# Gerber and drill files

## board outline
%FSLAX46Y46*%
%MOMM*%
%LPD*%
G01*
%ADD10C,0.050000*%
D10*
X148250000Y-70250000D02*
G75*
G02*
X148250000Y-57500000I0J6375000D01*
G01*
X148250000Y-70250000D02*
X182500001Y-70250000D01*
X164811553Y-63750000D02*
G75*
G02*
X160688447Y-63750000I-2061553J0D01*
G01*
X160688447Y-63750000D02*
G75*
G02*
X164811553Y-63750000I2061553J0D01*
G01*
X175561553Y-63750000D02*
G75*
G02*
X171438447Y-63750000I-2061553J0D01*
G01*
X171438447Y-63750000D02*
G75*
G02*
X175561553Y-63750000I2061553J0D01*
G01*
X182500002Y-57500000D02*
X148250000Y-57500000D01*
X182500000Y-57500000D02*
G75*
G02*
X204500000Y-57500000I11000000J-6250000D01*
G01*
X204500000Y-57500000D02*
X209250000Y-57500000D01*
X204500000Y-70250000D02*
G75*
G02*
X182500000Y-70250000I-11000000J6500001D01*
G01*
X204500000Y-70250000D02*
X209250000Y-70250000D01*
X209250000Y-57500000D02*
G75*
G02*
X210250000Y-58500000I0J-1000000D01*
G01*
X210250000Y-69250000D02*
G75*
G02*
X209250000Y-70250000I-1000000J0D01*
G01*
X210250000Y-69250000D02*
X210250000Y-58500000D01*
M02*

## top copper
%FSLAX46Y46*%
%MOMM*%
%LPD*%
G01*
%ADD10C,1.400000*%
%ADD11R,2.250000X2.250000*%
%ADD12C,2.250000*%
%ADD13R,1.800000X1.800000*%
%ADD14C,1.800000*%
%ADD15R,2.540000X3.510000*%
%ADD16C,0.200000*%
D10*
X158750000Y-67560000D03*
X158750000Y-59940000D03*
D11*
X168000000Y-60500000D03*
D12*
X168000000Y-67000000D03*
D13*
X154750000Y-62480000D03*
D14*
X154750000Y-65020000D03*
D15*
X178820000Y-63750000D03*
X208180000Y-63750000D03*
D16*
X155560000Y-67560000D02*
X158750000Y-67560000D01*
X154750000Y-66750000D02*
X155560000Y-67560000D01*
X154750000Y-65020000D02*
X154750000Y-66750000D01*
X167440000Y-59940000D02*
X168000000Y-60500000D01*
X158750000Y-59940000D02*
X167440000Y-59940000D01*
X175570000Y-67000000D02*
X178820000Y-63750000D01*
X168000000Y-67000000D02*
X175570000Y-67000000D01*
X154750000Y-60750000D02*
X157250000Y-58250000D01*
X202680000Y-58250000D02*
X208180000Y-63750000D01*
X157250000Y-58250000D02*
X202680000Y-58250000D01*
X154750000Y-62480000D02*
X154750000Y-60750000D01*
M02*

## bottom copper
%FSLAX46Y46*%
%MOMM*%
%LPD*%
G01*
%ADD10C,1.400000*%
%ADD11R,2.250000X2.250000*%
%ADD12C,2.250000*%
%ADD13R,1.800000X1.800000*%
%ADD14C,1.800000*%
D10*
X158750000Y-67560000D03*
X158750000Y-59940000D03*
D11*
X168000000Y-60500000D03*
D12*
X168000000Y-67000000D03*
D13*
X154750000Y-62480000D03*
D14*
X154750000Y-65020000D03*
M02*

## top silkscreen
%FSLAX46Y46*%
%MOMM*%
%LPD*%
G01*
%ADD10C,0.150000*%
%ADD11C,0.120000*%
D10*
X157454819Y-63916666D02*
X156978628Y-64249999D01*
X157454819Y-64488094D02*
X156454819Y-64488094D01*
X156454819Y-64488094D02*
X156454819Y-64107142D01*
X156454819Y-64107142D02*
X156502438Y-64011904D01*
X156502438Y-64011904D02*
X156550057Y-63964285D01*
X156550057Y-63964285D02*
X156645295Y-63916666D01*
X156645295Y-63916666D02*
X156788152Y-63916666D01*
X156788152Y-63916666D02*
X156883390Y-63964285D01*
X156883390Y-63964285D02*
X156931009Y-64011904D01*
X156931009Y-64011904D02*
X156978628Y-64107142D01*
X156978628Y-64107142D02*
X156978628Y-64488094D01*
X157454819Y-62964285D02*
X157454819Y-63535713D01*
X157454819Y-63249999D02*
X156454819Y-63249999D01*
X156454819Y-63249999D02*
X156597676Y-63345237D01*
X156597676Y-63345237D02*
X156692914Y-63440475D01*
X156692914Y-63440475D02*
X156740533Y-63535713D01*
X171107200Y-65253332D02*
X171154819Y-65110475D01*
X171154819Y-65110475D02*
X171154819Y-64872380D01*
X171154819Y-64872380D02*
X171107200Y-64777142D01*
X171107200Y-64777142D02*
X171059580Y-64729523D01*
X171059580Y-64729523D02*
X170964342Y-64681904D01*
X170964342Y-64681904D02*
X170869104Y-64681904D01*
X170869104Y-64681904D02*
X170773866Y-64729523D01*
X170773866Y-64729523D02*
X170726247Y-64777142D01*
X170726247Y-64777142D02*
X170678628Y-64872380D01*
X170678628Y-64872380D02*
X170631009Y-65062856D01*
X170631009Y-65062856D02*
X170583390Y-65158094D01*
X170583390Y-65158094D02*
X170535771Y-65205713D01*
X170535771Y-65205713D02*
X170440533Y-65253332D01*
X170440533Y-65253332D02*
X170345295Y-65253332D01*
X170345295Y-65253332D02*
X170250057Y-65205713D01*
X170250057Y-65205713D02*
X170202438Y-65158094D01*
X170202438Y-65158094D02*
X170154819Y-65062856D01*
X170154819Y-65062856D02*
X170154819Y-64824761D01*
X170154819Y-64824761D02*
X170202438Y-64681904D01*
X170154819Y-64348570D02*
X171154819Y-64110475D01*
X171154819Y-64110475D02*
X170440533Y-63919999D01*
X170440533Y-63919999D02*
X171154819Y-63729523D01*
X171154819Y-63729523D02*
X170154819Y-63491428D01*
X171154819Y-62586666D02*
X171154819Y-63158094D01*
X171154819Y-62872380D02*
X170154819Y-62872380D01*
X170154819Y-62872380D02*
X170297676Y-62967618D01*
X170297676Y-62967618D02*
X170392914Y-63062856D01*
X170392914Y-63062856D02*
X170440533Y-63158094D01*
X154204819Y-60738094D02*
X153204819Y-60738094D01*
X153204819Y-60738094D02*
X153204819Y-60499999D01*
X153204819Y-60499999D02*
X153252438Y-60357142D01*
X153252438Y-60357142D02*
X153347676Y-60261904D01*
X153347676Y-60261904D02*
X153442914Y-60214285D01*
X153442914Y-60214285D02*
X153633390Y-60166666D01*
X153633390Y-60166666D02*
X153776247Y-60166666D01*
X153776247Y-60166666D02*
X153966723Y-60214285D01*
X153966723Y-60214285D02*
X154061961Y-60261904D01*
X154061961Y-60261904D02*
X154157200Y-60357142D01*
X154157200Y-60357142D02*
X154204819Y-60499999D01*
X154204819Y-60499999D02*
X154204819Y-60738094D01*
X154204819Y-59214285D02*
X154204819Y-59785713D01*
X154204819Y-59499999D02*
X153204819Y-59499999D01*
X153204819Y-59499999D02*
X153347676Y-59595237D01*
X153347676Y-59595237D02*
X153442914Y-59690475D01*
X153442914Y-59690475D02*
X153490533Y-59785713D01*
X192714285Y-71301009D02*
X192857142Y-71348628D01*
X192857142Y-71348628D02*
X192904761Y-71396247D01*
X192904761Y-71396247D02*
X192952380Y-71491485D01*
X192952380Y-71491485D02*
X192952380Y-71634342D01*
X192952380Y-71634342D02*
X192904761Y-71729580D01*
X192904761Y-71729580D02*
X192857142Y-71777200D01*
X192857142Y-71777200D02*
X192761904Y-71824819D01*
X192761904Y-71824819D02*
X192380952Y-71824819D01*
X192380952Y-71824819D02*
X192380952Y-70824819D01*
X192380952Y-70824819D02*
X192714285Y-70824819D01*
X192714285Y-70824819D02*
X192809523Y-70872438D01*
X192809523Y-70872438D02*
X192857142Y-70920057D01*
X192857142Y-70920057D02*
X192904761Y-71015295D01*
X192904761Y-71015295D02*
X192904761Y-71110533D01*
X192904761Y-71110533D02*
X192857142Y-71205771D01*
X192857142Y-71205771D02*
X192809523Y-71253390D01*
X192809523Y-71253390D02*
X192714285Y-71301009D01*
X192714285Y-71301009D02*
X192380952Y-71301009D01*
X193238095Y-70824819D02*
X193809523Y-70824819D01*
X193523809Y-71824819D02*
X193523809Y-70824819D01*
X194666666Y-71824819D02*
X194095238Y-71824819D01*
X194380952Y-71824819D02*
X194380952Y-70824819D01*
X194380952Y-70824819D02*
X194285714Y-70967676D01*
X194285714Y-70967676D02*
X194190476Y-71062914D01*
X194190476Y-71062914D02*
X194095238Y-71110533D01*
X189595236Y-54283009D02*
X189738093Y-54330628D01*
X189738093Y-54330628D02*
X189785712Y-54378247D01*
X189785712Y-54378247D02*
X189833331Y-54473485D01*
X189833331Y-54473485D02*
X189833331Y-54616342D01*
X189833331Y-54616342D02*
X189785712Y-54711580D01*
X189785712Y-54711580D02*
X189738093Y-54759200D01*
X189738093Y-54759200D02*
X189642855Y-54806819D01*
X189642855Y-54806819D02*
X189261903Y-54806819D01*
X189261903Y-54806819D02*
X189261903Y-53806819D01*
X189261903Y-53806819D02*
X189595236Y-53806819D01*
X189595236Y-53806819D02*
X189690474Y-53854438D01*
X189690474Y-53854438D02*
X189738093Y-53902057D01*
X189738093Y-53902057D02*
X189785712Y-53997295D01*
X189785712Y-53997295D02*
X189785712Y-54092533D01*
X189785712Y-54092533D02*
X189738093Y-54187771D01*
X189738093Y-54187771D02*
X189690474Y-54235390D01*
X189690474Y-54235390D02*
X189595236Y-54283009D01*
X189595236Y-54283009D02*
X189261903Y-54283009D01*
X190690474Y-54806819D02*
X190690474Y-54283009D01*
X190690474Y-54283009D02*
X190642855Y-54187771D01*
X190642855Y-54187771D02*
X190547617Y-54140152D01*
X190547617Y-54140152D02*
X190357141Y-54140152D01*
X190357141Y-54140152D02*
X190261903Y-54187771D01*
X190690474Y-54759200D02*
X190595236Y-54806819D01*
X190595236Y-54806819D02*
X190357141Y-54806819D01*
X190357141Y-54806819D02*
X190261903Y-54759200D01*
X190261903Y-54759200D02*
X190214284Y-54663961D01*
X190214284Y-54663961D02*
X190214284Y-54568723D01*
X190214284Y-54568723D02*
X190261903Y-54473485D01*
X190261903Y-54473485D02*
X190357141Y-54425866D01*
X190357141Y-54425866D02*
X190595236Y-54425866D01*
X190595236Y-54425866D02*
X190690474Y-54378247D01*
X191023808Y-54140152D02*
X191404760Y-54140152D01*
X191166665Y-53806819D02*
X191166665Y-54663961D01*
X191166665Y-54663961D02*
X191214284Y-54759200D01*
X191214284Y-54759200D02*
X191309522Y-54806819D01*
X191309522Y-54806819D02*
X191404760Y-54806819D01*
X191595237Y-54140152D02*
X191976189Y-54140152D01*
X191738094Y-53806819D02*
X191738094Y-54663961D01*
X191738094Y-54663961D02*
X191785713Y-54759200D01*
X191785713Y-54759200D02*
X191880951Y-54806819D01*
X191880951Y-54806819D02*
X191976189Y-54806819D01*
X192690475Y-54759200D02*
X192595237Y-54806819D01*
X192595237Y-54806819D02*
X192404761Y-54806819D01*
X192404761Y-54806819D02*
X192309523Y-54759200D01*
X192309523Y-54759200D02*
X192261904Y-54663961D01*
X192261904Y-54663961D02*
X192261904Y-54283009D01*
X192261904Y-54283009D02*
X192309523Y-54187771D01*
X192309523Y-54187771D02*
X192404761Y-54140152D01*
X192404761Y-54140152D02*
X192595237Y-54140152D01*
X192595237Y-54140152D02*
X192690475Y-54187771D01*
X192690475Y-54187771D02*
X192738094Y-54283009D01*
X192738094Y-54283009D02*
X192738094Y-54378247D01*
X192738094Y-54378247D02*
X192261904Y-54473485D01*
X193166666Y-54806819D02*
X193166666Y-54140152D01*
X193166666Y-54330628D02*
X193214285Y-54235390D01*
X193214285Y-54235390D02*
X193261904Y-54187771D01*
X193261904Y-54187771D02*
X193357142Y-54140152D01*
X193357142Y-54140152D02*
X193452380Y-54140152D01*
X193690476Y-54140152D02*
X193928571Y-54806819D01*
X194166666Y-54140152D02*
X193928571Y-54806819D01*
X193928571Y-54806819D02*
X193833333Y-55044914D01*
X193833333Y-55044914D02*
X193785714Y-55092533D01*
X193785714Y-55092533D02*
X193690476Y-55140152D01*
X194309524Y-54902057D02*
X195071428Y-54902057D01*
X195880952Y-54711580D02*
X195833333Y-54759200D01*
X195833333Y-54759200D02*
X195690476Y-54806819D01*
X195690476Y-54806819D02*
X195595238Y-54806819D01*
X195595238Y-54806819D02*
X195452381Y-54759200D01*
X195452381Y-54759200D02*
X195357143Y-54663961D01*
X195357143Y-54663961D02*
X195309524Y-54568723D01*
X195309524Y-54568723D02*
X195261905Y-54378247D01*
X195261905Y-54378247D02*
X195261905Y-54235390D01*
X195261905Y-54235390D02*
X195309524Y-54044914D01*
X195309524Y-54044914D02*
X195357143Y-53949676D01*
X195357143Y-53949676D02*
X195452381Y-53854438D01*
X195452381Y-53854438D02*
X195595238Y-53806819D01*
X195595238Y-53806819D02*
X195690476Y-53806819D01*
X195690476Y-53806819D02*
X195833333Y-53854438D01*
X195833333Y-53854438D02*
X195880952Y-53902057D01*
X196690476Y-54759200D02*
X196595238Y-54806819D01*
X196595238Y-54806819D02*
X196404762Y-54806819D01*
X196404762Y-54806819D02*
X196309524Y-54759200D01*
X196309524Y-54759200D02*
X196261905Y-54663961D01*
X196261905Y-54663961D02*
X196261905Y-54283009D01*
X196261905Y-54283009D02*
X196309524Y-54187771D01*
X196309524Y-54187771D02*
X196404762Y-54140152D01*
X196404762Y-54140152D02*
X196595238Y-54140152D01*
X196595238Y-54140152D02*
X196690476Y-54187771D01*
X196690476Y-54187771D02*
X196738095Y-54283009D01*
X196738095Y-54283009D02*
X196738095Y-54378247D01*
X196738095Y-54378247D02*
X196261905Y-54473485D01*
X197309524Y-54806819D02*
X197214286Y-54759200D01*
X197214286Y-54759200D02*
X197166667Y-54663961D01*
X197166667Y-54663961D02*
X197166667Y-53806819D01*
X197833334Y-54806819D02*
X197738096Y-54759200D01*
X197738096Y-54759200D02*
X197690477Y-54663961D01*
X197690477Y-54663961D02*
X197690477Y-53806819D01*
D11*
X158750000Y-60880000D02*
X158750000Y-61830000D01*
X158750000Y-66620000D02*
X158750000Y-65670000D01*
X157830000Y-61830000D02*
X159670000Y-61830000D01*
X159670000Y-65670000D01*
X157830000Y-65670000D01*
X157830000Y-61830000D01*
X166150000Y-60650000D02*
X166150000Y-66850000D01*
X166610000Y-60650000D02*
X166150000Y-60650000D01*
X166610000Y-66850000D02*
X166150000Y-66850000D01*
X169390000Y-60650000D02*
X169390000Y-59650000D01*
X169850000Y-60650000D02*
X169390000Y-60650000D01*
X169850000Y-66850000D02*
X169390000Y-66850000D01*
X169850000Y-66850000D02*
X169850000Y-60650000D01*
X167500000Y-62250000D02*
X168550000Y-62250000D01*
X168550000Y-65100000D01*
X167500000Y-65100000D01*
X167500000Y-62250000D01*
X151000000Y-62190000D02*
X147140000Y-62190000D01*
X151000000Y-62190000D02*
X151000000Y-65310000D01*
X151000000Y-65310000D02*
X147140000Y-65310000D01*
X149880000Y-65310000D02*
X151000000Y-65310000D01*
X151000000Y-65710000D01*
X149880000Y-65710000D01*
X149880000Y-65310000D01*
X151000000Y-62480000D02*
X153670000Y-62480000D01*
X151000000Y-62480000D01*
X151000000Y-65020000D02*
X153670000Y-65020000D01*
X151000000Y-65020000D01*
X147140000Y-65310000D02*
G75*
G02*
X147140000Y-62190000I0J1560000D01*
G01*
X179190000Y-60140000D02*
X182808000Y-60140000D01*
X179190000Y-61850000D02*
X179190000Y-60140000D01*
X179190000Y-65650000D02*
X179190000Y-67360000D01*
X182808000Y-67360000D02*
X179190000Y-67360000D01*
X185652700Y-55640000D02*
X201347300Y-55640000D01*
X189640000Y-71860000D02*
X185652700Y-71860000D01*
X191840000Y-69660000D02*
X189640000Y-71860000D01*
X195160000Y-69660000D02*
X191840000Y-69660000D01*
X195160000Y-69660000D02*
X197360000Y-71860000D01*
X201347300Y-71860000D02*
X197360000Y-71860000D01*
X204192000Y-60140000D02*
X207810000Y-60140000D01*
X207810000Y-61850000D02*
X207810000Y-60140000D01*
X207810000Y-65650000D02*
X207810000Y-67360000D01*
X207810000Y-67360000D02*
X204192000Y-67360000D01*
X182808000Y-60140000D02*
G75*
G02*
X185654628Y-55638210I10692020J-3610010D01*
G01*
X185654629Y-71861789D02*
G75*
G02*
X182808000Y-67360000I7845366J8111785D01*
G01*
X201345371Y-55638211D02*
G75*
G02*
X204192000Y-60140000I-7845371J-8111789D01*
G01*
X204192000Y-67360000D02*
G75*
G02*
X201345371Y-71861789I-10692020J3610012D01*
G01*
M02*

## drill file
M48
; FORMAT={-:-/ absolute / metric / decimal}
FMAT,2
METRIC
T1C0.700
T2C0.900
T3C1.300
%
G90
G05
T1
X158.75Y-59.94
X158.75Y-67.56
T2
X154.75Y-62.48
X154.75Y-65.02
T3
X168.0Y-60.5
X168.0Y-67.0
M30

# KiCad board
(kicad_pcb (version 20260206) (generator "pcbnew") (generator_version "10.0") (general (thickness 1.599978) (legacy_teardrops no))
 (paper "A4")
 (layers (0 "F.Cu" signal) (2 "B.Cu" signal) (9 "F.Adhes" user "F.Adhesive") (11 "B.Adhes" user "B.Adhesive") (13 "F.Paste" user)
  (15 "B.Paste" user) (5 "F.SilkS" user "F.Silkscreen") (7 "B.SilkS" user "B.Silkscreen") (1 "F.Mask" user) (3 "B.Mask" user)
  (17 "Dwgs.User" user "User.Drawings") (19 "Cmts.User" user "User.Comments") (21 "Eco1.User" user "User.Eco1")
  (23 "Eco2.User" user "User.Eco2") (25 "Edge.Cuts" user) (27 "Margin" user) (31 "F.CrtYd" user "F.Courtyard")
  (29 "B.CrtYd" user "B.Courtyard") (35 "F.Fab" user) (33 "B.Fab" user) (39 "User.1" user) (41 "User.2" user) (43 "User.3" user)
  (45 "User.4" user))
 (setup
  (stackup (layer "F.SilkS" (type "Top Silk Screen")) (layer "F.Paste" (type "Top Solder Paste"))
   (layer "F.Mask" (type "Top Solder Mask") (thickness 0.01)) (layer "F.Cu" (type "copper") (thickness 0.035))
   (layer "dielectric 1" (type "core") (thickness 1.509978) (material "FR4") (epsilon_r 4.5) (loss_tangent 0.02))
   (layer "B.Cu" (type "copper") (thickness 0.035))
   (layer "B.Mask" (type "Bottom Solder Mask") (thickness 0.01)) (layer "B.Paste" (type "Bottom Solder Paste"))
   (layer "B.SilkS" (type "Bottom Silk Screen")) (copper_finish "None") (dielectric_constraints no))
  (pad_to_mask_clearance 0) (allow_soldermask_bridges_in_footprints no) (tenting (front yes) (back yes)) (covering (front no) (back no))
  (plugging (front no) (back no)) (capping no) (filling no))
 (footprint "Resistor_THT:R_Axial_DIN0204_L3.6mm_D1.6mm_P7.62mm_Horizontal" (layer "F.Cu") (at 158.75 67.56 90)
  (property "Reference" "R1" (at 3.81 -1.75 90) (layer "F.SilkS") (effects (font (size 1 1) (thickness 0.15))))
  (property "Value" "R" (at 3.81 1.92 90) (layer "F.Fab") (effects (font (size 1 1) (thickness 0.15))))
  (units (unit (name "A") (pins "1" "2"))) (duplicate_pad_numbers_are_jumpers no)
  (fp_line (start 6.68 0) (end 5.73 0) (stroke (width 0.12) (type solid)) (layer "F.SilkS"))
  (fp_line (start 0.94 0) (end 1.89 0) (stroke (width 0.12) (type solid)) (layer "F.SilkS"))
  (fp_rect (start 1.89 -0.92) (end 5.73 0.92) (stroke (width 0.12) (type solid)) (fill no) (layer "F.SilkS"))
  (pad "1" thru_hole circle (at 0 0 90) (size 1.4 1.4) (drill 0.7) (layers "*.Cu" "*.Mask") (remove_unused_layers no) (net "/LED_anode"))
  (pad "2" thru_hole circle (at 7.62 0 90) (size 1.4 1.4) (drill 0.7) (layers "*.Cu" "*.Mask") (remove_unused_layers no)
   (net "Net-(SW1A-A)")))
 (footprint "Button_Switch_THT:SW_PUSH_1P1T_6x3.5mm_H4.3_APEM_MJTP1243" (layer "F.Cu") (at 168 60.5 -90)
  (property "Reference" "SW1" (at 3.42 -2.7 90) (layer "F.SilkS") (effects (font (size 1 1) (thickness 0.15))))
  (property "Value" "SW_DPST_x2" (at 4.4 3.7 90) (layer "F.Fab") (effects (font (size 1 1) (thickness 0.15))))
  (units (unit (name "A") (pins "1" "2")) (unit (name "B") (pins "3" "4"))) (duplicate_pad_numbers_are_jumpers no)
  (fp_line (start 0.15 1.85) (end 6.35 1.85) (stroke (width 0.12) (type solid)) (layer "F.SilkS"))
  (fp_line (start 0.15 1.39) (end 0.15 1.85) (stroke (width 0.12) (type solid)) (layer "F.SilkS"))
  (fp_line (start 6.35 1.39) (end 6.35 1.85) (stroke (width 0.12) (type solid)) (layer "F.SilkS"))
  (fp_line (start 0.15 -1.39) (end -0.85 -1.39) (stroke (width 0.12) (type default)) (layer "F.SilkS"))
  (fp_line (start 0.15 -1.85) (end 0.15 -1.39) (stroke (width 0.12) (type default)) (layer "F.SilkS"))
  (fp_line (start 6.35 -1.85) (end 6.35 -1.39) (stroke (width 0.12) (type solid)) (layer "F.SilkS"))
  (fp_line (start 6.35 -1.85) (end 0.15 -1.85) (stroke (width 0.12) (type solid)) (layer "F.SilkS"))
  (fp_rect (start 1.75 -0.55) (end 4.6 0.5) (stroke (width 0.12) (type default)) (fill no) (layer "F.SilkS"))
  (pad "1" thru_hole rect (at 0 0) (size 2.25 2.25) (drill 1.3) (layers "*.Cu" "*.Mask") (remove_unused_layers no) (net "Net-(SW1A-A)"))
  (pad "2" thru_hole circle (at 6.5 0) (size 2.25 2.25) (drill 1.3) (layers "*.Cu" "*.Mask") (remove_unused_layers no) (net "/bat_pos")))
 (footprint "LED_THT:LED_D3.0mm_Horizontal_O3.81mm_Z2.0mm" (layer "F.Cu") (at 154.75 62.48 -90)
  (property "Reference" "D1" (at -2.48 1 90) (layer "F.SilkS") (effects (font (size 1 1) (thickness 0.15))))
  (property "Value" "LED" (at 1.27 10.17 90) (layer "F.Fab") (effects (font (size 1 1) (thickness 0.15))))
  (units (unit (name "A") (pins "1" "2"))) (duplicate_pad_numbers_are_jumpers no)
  (fp_line (start -0.29 3.75) (end -0.29 7.61) (stroke (width 0.12) (type solid)) (layer "F.SilkS"))
  (fp_line (start -0.29 3.75) (end 2.83 3.75) (stroke (width 0.12) (type solid)) (layer "F.SilkS"))
  (fp_line (start 2.83 3.75) (end 2.83 7.61) (stroke (width 0.12) (type solid)) (layer "F.SilkS"))
  (fp_rect (start 2.83 3.75) (end 3.23 4.87) (stroke (width 0.12) (type solid)) (fill no) (layer "F.SilkS"))
  (fp_rect (start 0 1.08) (end 0 3.75) (stroke (width 0.12) (type solid)) (fill no) (layer "F.SilkS"))
  (fp_rect (start 2.54 1.08) (end 2.54 3.75) (stroke (width 0.12) (type solid)) (fill no) (layer "F.SilkS"))
  (fp_arc (start 2.83 7.61) (mid 1.27 9.17) (end -0.29 7.61) (stroke (width 0.12) (type solid)) (layer "F.SilkS"))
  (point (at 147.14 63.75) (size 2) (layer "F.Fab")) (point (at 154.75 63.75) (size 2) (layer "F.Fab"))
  (pad "1" thru_hole rect (at 0 0 270) (size 1.8 1.8) (drill 0.9) (layers "*.Cu" "*.Mask") (remove_unused_layers no) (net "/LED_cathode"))
  (pad "2" thru_hole circle (at 2.54 0 270) (size 1.8 1.8) (drill 0.9) (layers "*.Cu" "*.Mask") (remove_unused_layers no) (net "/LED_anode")))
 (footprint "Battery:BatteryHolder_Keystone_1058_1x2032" (layer "F.Cu") (at 193.5 63.75)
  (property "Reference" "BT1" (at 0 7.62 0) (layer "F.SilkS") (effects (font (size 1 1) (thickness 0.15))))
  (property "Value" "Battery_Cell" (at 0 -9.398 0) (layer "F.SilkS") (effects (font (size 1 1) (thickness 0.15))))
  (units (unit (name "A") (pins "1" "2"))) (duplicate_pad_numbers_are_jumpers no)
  (fp_line (start -14.31 -3.61) (end -10.692 -3.61) (stroke (width 0.12) (type solid)) (layer "F.SilkS"))
  (fp_line (start -14.31 -1.9) (end -14.31 -3.61) (stroke (width 0.12) (type solid)) (layer "F.SilkS"))
  (fp_line (start -14.31 1.9) (end -14.31 3.61) (stroke (width 0.12) (type solid)) (layer "F.SilkS"))
  (fp_line (start -10.692 3.61) (end -14.31 3.61) (stroke (width 0.12) (type solid)) (layer "F.SilkS"))
  (fp_line (start -7.8473 -8.11) (end 7.8473 -8.11) (stroke (width 0.12) (type solid)) (layer "F.SilkS"))
  (fp_line (start -3.86 8.11) (end -7.8473 8.11) (stroke (width 0.12) (type solid)) (layer "F.SilkS"))
  (fp_line (start -1.66 5.91) (end -3.86 8.11) (stroke (width 0.12) (type solid)) (layer "F.SilkS"))
  (fp_line (start 1.66 5.91) (end -1.66 5.91) (stroke (width 0.12) (type solid)) (layer "F.SilkS"))
  (fp_line (start 1.66 5.91) (end 3.86 8.11) (stroke (width 0.12) (type solid)) (layer "F.SilkS"))
  (fp_line (start 7.8473 8.11) (end 3.86 8.11) (stroke (width 0.12) (type solid)) (layer "F.SilkS"))
  (fp_line (start 10.692 -3.61) (end 14.31 -3.61) (stroke (width 0.12) (type solid)) (layer "F.SilkS"))
  (fp_line (start 14.31 -1.9) (end 14.31 -3.61) (stroke (width 0.12) (type solid)) (layer "F.SilkS"))
  (fp_line (start 14.31 1.9) (end 14.31 3.61) (stroke (width 0.12) (type solid)) (layer "F.SilkS"))
  (fp_line (start 14.31 3.61) (end 10.692 3.61) (stroke (width 0.12) (type solid)) (layer "F.SilkS"))
  (fp_arc (start -10.692 -3.61) (mid -9.538084 -6.031244) (end -7.845371 -8.111789) (stroke (width 0.12) (type solid)) (layer "F.SilkS"))
  (fp_arc (start -7.845371 8.111789) (mid -9.538085 6.031244) (end -10.692 3.61) (stroke (width 0.12) (type solid)) (layer "F.SilkS"))
  (fp_arc (start 7.845371 -8.111789) (mid 9.538085 -6.031244) (end 10.692 -3.61) (stroke (width 0.12) (type solid)) (layer "F.SilkS"))
  (fp_arc (start 10.692 3.61) (mid 9.538084 6.031244) (end 7.845371 8.111789) (stroke (width 0.12) (type solid)) (layer "F.SilkS"))
  (pad "1" smd rect (at -14.68 0) (size 2.54 3.51) (layers "F.Cu" "F.Mask" "F.Paste") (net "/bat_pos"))
  (pad "2" smd rect (at 14.68 0) (size 2.54 3.51) (layers "F.Cu" "F.Mask" "F.Paste") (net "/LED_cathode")))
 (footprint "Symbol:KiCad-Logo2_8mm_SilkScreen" (layer "B.Cu") (at 193.75 62.75 180)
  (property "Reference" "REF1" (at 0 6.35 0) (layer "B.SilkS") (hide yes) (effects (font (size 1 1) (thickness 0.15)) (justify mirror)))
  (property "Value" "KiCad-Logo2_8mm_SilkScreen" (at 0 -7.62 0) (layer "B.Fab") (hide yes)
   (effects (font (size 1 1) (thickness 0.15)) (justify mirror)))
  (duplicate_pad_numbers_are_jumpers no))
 (gr_arc (start 148.25 70.25) (mid 141.875 63.875) (end 148.25 57.5) (stroke (width 0.05) (type default)) (layer "Edge.Cuts"))
 (gr_line (start 148.25 70.25) (end 182.500001 70.25) (stroke (width 0.05) (type default)) (layer "Edge.Cuts"))
 (gr_circle (center 162.75 63.75) (end 164.75 64.25) (stroke (width 0.05) (type default)) (fill no) (layer "Edge.Cuts"))
 (gr_circle (center 173.5 63.75) (end 175.5 64.25) (stroke (width 0.05) (type default)) (fill no) (layer "Edge.Cuts"))
 (gr_line (start 182.500002 57.5) (end 148.25 57.5) (stroke (width 0.05) (type default)) (layer "Edge.Cuts"))
 (gr_arc (start 182.5 57.5) (mid 193.5 51.098419) (end 204.5 57.5) (stroke (width 0.05) (type default)) (layer "Edge.Cuts"))
 (gr_line (start 204.5 57.5) (end 209.25 57.5) (stroke (width 0.05) (type default)) (layer "Edge.Cuts"))
 (gr_arc (start 204.5 70.25) (mid 193.5 76.526932) (end 182.5 70.25) (stroke (width 0.05) (type default)) (layer "Edge.Cuts"))
 (gr_line (start 204.5 70.25) (end 209.25 70.25) (stroke (width 0.05) (type default)) (layer "Edge.Cuts"))
 (gr_arc (start 209.25 57.5) (mid 209.957107 57.792893) (end 210.25 58.5) (stroke (width 0.05) (type default)) (layer "Edge.Cuts"))
 (gr_arc (start 210.25 69.25) (mid 209.957107 69.957107) (end 209.25 70.25) (stroke (width 0.05) (type default)) (layer "Edge.Cuts"))
 (gr_line (start 210.25 69.25) (end 210.25 58.5) (stroke (width 0.05) (type default)) (layer "Edge.Cuts"))
 (segment (start 155.56 67.56) (end 158.75 67.56) (width 0.2) (layer "F.Cu") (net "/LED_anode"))
 (segment (start 154.75 66.75) (end 155.56 67.56) (width 0.2) (layer "F.Cu") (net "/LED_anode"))
 (segment (start 154.75 65.02) (end 154.75 66.75) (width 0.2) (layer "F.Cu") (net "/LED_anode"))
 (segment (start 167.44 59.94) (end 168 60.5) (width 0.2) (layer "F.Cu") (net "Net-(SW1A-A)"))
 (segment (start 158.75 59.94) (end 167.44 59.94) (width 0.2) (layer "F.Cu") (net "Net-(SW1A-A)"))
 (segment (start 175.57 67) (end 178.82 63.75) (width 0.2) (layer "F.Cu") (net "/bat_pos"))
 (segment (start 168 67) (end 175.57 67) (width 0.2) (layer "F.Cu") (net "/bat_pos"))
 (segment (start 154.75 60.75) (end 157.25 58.25) (width 0.2) (layer "F.Cu") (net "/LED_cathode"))
 (segment (start 202.68 58.25) (end 208.18 63.75) (width 0.2) (layer "F.Cu") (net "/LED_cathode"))
 (segment (start 157.25 58.25) (end 202.68 58.25) (width 0.2) (layer "F.Cu") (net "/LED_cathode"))
 (segment (start 154.75 62.48) (end 154.75 60.75) (width 0.2) (layer "F.Cu") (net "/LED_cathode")))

